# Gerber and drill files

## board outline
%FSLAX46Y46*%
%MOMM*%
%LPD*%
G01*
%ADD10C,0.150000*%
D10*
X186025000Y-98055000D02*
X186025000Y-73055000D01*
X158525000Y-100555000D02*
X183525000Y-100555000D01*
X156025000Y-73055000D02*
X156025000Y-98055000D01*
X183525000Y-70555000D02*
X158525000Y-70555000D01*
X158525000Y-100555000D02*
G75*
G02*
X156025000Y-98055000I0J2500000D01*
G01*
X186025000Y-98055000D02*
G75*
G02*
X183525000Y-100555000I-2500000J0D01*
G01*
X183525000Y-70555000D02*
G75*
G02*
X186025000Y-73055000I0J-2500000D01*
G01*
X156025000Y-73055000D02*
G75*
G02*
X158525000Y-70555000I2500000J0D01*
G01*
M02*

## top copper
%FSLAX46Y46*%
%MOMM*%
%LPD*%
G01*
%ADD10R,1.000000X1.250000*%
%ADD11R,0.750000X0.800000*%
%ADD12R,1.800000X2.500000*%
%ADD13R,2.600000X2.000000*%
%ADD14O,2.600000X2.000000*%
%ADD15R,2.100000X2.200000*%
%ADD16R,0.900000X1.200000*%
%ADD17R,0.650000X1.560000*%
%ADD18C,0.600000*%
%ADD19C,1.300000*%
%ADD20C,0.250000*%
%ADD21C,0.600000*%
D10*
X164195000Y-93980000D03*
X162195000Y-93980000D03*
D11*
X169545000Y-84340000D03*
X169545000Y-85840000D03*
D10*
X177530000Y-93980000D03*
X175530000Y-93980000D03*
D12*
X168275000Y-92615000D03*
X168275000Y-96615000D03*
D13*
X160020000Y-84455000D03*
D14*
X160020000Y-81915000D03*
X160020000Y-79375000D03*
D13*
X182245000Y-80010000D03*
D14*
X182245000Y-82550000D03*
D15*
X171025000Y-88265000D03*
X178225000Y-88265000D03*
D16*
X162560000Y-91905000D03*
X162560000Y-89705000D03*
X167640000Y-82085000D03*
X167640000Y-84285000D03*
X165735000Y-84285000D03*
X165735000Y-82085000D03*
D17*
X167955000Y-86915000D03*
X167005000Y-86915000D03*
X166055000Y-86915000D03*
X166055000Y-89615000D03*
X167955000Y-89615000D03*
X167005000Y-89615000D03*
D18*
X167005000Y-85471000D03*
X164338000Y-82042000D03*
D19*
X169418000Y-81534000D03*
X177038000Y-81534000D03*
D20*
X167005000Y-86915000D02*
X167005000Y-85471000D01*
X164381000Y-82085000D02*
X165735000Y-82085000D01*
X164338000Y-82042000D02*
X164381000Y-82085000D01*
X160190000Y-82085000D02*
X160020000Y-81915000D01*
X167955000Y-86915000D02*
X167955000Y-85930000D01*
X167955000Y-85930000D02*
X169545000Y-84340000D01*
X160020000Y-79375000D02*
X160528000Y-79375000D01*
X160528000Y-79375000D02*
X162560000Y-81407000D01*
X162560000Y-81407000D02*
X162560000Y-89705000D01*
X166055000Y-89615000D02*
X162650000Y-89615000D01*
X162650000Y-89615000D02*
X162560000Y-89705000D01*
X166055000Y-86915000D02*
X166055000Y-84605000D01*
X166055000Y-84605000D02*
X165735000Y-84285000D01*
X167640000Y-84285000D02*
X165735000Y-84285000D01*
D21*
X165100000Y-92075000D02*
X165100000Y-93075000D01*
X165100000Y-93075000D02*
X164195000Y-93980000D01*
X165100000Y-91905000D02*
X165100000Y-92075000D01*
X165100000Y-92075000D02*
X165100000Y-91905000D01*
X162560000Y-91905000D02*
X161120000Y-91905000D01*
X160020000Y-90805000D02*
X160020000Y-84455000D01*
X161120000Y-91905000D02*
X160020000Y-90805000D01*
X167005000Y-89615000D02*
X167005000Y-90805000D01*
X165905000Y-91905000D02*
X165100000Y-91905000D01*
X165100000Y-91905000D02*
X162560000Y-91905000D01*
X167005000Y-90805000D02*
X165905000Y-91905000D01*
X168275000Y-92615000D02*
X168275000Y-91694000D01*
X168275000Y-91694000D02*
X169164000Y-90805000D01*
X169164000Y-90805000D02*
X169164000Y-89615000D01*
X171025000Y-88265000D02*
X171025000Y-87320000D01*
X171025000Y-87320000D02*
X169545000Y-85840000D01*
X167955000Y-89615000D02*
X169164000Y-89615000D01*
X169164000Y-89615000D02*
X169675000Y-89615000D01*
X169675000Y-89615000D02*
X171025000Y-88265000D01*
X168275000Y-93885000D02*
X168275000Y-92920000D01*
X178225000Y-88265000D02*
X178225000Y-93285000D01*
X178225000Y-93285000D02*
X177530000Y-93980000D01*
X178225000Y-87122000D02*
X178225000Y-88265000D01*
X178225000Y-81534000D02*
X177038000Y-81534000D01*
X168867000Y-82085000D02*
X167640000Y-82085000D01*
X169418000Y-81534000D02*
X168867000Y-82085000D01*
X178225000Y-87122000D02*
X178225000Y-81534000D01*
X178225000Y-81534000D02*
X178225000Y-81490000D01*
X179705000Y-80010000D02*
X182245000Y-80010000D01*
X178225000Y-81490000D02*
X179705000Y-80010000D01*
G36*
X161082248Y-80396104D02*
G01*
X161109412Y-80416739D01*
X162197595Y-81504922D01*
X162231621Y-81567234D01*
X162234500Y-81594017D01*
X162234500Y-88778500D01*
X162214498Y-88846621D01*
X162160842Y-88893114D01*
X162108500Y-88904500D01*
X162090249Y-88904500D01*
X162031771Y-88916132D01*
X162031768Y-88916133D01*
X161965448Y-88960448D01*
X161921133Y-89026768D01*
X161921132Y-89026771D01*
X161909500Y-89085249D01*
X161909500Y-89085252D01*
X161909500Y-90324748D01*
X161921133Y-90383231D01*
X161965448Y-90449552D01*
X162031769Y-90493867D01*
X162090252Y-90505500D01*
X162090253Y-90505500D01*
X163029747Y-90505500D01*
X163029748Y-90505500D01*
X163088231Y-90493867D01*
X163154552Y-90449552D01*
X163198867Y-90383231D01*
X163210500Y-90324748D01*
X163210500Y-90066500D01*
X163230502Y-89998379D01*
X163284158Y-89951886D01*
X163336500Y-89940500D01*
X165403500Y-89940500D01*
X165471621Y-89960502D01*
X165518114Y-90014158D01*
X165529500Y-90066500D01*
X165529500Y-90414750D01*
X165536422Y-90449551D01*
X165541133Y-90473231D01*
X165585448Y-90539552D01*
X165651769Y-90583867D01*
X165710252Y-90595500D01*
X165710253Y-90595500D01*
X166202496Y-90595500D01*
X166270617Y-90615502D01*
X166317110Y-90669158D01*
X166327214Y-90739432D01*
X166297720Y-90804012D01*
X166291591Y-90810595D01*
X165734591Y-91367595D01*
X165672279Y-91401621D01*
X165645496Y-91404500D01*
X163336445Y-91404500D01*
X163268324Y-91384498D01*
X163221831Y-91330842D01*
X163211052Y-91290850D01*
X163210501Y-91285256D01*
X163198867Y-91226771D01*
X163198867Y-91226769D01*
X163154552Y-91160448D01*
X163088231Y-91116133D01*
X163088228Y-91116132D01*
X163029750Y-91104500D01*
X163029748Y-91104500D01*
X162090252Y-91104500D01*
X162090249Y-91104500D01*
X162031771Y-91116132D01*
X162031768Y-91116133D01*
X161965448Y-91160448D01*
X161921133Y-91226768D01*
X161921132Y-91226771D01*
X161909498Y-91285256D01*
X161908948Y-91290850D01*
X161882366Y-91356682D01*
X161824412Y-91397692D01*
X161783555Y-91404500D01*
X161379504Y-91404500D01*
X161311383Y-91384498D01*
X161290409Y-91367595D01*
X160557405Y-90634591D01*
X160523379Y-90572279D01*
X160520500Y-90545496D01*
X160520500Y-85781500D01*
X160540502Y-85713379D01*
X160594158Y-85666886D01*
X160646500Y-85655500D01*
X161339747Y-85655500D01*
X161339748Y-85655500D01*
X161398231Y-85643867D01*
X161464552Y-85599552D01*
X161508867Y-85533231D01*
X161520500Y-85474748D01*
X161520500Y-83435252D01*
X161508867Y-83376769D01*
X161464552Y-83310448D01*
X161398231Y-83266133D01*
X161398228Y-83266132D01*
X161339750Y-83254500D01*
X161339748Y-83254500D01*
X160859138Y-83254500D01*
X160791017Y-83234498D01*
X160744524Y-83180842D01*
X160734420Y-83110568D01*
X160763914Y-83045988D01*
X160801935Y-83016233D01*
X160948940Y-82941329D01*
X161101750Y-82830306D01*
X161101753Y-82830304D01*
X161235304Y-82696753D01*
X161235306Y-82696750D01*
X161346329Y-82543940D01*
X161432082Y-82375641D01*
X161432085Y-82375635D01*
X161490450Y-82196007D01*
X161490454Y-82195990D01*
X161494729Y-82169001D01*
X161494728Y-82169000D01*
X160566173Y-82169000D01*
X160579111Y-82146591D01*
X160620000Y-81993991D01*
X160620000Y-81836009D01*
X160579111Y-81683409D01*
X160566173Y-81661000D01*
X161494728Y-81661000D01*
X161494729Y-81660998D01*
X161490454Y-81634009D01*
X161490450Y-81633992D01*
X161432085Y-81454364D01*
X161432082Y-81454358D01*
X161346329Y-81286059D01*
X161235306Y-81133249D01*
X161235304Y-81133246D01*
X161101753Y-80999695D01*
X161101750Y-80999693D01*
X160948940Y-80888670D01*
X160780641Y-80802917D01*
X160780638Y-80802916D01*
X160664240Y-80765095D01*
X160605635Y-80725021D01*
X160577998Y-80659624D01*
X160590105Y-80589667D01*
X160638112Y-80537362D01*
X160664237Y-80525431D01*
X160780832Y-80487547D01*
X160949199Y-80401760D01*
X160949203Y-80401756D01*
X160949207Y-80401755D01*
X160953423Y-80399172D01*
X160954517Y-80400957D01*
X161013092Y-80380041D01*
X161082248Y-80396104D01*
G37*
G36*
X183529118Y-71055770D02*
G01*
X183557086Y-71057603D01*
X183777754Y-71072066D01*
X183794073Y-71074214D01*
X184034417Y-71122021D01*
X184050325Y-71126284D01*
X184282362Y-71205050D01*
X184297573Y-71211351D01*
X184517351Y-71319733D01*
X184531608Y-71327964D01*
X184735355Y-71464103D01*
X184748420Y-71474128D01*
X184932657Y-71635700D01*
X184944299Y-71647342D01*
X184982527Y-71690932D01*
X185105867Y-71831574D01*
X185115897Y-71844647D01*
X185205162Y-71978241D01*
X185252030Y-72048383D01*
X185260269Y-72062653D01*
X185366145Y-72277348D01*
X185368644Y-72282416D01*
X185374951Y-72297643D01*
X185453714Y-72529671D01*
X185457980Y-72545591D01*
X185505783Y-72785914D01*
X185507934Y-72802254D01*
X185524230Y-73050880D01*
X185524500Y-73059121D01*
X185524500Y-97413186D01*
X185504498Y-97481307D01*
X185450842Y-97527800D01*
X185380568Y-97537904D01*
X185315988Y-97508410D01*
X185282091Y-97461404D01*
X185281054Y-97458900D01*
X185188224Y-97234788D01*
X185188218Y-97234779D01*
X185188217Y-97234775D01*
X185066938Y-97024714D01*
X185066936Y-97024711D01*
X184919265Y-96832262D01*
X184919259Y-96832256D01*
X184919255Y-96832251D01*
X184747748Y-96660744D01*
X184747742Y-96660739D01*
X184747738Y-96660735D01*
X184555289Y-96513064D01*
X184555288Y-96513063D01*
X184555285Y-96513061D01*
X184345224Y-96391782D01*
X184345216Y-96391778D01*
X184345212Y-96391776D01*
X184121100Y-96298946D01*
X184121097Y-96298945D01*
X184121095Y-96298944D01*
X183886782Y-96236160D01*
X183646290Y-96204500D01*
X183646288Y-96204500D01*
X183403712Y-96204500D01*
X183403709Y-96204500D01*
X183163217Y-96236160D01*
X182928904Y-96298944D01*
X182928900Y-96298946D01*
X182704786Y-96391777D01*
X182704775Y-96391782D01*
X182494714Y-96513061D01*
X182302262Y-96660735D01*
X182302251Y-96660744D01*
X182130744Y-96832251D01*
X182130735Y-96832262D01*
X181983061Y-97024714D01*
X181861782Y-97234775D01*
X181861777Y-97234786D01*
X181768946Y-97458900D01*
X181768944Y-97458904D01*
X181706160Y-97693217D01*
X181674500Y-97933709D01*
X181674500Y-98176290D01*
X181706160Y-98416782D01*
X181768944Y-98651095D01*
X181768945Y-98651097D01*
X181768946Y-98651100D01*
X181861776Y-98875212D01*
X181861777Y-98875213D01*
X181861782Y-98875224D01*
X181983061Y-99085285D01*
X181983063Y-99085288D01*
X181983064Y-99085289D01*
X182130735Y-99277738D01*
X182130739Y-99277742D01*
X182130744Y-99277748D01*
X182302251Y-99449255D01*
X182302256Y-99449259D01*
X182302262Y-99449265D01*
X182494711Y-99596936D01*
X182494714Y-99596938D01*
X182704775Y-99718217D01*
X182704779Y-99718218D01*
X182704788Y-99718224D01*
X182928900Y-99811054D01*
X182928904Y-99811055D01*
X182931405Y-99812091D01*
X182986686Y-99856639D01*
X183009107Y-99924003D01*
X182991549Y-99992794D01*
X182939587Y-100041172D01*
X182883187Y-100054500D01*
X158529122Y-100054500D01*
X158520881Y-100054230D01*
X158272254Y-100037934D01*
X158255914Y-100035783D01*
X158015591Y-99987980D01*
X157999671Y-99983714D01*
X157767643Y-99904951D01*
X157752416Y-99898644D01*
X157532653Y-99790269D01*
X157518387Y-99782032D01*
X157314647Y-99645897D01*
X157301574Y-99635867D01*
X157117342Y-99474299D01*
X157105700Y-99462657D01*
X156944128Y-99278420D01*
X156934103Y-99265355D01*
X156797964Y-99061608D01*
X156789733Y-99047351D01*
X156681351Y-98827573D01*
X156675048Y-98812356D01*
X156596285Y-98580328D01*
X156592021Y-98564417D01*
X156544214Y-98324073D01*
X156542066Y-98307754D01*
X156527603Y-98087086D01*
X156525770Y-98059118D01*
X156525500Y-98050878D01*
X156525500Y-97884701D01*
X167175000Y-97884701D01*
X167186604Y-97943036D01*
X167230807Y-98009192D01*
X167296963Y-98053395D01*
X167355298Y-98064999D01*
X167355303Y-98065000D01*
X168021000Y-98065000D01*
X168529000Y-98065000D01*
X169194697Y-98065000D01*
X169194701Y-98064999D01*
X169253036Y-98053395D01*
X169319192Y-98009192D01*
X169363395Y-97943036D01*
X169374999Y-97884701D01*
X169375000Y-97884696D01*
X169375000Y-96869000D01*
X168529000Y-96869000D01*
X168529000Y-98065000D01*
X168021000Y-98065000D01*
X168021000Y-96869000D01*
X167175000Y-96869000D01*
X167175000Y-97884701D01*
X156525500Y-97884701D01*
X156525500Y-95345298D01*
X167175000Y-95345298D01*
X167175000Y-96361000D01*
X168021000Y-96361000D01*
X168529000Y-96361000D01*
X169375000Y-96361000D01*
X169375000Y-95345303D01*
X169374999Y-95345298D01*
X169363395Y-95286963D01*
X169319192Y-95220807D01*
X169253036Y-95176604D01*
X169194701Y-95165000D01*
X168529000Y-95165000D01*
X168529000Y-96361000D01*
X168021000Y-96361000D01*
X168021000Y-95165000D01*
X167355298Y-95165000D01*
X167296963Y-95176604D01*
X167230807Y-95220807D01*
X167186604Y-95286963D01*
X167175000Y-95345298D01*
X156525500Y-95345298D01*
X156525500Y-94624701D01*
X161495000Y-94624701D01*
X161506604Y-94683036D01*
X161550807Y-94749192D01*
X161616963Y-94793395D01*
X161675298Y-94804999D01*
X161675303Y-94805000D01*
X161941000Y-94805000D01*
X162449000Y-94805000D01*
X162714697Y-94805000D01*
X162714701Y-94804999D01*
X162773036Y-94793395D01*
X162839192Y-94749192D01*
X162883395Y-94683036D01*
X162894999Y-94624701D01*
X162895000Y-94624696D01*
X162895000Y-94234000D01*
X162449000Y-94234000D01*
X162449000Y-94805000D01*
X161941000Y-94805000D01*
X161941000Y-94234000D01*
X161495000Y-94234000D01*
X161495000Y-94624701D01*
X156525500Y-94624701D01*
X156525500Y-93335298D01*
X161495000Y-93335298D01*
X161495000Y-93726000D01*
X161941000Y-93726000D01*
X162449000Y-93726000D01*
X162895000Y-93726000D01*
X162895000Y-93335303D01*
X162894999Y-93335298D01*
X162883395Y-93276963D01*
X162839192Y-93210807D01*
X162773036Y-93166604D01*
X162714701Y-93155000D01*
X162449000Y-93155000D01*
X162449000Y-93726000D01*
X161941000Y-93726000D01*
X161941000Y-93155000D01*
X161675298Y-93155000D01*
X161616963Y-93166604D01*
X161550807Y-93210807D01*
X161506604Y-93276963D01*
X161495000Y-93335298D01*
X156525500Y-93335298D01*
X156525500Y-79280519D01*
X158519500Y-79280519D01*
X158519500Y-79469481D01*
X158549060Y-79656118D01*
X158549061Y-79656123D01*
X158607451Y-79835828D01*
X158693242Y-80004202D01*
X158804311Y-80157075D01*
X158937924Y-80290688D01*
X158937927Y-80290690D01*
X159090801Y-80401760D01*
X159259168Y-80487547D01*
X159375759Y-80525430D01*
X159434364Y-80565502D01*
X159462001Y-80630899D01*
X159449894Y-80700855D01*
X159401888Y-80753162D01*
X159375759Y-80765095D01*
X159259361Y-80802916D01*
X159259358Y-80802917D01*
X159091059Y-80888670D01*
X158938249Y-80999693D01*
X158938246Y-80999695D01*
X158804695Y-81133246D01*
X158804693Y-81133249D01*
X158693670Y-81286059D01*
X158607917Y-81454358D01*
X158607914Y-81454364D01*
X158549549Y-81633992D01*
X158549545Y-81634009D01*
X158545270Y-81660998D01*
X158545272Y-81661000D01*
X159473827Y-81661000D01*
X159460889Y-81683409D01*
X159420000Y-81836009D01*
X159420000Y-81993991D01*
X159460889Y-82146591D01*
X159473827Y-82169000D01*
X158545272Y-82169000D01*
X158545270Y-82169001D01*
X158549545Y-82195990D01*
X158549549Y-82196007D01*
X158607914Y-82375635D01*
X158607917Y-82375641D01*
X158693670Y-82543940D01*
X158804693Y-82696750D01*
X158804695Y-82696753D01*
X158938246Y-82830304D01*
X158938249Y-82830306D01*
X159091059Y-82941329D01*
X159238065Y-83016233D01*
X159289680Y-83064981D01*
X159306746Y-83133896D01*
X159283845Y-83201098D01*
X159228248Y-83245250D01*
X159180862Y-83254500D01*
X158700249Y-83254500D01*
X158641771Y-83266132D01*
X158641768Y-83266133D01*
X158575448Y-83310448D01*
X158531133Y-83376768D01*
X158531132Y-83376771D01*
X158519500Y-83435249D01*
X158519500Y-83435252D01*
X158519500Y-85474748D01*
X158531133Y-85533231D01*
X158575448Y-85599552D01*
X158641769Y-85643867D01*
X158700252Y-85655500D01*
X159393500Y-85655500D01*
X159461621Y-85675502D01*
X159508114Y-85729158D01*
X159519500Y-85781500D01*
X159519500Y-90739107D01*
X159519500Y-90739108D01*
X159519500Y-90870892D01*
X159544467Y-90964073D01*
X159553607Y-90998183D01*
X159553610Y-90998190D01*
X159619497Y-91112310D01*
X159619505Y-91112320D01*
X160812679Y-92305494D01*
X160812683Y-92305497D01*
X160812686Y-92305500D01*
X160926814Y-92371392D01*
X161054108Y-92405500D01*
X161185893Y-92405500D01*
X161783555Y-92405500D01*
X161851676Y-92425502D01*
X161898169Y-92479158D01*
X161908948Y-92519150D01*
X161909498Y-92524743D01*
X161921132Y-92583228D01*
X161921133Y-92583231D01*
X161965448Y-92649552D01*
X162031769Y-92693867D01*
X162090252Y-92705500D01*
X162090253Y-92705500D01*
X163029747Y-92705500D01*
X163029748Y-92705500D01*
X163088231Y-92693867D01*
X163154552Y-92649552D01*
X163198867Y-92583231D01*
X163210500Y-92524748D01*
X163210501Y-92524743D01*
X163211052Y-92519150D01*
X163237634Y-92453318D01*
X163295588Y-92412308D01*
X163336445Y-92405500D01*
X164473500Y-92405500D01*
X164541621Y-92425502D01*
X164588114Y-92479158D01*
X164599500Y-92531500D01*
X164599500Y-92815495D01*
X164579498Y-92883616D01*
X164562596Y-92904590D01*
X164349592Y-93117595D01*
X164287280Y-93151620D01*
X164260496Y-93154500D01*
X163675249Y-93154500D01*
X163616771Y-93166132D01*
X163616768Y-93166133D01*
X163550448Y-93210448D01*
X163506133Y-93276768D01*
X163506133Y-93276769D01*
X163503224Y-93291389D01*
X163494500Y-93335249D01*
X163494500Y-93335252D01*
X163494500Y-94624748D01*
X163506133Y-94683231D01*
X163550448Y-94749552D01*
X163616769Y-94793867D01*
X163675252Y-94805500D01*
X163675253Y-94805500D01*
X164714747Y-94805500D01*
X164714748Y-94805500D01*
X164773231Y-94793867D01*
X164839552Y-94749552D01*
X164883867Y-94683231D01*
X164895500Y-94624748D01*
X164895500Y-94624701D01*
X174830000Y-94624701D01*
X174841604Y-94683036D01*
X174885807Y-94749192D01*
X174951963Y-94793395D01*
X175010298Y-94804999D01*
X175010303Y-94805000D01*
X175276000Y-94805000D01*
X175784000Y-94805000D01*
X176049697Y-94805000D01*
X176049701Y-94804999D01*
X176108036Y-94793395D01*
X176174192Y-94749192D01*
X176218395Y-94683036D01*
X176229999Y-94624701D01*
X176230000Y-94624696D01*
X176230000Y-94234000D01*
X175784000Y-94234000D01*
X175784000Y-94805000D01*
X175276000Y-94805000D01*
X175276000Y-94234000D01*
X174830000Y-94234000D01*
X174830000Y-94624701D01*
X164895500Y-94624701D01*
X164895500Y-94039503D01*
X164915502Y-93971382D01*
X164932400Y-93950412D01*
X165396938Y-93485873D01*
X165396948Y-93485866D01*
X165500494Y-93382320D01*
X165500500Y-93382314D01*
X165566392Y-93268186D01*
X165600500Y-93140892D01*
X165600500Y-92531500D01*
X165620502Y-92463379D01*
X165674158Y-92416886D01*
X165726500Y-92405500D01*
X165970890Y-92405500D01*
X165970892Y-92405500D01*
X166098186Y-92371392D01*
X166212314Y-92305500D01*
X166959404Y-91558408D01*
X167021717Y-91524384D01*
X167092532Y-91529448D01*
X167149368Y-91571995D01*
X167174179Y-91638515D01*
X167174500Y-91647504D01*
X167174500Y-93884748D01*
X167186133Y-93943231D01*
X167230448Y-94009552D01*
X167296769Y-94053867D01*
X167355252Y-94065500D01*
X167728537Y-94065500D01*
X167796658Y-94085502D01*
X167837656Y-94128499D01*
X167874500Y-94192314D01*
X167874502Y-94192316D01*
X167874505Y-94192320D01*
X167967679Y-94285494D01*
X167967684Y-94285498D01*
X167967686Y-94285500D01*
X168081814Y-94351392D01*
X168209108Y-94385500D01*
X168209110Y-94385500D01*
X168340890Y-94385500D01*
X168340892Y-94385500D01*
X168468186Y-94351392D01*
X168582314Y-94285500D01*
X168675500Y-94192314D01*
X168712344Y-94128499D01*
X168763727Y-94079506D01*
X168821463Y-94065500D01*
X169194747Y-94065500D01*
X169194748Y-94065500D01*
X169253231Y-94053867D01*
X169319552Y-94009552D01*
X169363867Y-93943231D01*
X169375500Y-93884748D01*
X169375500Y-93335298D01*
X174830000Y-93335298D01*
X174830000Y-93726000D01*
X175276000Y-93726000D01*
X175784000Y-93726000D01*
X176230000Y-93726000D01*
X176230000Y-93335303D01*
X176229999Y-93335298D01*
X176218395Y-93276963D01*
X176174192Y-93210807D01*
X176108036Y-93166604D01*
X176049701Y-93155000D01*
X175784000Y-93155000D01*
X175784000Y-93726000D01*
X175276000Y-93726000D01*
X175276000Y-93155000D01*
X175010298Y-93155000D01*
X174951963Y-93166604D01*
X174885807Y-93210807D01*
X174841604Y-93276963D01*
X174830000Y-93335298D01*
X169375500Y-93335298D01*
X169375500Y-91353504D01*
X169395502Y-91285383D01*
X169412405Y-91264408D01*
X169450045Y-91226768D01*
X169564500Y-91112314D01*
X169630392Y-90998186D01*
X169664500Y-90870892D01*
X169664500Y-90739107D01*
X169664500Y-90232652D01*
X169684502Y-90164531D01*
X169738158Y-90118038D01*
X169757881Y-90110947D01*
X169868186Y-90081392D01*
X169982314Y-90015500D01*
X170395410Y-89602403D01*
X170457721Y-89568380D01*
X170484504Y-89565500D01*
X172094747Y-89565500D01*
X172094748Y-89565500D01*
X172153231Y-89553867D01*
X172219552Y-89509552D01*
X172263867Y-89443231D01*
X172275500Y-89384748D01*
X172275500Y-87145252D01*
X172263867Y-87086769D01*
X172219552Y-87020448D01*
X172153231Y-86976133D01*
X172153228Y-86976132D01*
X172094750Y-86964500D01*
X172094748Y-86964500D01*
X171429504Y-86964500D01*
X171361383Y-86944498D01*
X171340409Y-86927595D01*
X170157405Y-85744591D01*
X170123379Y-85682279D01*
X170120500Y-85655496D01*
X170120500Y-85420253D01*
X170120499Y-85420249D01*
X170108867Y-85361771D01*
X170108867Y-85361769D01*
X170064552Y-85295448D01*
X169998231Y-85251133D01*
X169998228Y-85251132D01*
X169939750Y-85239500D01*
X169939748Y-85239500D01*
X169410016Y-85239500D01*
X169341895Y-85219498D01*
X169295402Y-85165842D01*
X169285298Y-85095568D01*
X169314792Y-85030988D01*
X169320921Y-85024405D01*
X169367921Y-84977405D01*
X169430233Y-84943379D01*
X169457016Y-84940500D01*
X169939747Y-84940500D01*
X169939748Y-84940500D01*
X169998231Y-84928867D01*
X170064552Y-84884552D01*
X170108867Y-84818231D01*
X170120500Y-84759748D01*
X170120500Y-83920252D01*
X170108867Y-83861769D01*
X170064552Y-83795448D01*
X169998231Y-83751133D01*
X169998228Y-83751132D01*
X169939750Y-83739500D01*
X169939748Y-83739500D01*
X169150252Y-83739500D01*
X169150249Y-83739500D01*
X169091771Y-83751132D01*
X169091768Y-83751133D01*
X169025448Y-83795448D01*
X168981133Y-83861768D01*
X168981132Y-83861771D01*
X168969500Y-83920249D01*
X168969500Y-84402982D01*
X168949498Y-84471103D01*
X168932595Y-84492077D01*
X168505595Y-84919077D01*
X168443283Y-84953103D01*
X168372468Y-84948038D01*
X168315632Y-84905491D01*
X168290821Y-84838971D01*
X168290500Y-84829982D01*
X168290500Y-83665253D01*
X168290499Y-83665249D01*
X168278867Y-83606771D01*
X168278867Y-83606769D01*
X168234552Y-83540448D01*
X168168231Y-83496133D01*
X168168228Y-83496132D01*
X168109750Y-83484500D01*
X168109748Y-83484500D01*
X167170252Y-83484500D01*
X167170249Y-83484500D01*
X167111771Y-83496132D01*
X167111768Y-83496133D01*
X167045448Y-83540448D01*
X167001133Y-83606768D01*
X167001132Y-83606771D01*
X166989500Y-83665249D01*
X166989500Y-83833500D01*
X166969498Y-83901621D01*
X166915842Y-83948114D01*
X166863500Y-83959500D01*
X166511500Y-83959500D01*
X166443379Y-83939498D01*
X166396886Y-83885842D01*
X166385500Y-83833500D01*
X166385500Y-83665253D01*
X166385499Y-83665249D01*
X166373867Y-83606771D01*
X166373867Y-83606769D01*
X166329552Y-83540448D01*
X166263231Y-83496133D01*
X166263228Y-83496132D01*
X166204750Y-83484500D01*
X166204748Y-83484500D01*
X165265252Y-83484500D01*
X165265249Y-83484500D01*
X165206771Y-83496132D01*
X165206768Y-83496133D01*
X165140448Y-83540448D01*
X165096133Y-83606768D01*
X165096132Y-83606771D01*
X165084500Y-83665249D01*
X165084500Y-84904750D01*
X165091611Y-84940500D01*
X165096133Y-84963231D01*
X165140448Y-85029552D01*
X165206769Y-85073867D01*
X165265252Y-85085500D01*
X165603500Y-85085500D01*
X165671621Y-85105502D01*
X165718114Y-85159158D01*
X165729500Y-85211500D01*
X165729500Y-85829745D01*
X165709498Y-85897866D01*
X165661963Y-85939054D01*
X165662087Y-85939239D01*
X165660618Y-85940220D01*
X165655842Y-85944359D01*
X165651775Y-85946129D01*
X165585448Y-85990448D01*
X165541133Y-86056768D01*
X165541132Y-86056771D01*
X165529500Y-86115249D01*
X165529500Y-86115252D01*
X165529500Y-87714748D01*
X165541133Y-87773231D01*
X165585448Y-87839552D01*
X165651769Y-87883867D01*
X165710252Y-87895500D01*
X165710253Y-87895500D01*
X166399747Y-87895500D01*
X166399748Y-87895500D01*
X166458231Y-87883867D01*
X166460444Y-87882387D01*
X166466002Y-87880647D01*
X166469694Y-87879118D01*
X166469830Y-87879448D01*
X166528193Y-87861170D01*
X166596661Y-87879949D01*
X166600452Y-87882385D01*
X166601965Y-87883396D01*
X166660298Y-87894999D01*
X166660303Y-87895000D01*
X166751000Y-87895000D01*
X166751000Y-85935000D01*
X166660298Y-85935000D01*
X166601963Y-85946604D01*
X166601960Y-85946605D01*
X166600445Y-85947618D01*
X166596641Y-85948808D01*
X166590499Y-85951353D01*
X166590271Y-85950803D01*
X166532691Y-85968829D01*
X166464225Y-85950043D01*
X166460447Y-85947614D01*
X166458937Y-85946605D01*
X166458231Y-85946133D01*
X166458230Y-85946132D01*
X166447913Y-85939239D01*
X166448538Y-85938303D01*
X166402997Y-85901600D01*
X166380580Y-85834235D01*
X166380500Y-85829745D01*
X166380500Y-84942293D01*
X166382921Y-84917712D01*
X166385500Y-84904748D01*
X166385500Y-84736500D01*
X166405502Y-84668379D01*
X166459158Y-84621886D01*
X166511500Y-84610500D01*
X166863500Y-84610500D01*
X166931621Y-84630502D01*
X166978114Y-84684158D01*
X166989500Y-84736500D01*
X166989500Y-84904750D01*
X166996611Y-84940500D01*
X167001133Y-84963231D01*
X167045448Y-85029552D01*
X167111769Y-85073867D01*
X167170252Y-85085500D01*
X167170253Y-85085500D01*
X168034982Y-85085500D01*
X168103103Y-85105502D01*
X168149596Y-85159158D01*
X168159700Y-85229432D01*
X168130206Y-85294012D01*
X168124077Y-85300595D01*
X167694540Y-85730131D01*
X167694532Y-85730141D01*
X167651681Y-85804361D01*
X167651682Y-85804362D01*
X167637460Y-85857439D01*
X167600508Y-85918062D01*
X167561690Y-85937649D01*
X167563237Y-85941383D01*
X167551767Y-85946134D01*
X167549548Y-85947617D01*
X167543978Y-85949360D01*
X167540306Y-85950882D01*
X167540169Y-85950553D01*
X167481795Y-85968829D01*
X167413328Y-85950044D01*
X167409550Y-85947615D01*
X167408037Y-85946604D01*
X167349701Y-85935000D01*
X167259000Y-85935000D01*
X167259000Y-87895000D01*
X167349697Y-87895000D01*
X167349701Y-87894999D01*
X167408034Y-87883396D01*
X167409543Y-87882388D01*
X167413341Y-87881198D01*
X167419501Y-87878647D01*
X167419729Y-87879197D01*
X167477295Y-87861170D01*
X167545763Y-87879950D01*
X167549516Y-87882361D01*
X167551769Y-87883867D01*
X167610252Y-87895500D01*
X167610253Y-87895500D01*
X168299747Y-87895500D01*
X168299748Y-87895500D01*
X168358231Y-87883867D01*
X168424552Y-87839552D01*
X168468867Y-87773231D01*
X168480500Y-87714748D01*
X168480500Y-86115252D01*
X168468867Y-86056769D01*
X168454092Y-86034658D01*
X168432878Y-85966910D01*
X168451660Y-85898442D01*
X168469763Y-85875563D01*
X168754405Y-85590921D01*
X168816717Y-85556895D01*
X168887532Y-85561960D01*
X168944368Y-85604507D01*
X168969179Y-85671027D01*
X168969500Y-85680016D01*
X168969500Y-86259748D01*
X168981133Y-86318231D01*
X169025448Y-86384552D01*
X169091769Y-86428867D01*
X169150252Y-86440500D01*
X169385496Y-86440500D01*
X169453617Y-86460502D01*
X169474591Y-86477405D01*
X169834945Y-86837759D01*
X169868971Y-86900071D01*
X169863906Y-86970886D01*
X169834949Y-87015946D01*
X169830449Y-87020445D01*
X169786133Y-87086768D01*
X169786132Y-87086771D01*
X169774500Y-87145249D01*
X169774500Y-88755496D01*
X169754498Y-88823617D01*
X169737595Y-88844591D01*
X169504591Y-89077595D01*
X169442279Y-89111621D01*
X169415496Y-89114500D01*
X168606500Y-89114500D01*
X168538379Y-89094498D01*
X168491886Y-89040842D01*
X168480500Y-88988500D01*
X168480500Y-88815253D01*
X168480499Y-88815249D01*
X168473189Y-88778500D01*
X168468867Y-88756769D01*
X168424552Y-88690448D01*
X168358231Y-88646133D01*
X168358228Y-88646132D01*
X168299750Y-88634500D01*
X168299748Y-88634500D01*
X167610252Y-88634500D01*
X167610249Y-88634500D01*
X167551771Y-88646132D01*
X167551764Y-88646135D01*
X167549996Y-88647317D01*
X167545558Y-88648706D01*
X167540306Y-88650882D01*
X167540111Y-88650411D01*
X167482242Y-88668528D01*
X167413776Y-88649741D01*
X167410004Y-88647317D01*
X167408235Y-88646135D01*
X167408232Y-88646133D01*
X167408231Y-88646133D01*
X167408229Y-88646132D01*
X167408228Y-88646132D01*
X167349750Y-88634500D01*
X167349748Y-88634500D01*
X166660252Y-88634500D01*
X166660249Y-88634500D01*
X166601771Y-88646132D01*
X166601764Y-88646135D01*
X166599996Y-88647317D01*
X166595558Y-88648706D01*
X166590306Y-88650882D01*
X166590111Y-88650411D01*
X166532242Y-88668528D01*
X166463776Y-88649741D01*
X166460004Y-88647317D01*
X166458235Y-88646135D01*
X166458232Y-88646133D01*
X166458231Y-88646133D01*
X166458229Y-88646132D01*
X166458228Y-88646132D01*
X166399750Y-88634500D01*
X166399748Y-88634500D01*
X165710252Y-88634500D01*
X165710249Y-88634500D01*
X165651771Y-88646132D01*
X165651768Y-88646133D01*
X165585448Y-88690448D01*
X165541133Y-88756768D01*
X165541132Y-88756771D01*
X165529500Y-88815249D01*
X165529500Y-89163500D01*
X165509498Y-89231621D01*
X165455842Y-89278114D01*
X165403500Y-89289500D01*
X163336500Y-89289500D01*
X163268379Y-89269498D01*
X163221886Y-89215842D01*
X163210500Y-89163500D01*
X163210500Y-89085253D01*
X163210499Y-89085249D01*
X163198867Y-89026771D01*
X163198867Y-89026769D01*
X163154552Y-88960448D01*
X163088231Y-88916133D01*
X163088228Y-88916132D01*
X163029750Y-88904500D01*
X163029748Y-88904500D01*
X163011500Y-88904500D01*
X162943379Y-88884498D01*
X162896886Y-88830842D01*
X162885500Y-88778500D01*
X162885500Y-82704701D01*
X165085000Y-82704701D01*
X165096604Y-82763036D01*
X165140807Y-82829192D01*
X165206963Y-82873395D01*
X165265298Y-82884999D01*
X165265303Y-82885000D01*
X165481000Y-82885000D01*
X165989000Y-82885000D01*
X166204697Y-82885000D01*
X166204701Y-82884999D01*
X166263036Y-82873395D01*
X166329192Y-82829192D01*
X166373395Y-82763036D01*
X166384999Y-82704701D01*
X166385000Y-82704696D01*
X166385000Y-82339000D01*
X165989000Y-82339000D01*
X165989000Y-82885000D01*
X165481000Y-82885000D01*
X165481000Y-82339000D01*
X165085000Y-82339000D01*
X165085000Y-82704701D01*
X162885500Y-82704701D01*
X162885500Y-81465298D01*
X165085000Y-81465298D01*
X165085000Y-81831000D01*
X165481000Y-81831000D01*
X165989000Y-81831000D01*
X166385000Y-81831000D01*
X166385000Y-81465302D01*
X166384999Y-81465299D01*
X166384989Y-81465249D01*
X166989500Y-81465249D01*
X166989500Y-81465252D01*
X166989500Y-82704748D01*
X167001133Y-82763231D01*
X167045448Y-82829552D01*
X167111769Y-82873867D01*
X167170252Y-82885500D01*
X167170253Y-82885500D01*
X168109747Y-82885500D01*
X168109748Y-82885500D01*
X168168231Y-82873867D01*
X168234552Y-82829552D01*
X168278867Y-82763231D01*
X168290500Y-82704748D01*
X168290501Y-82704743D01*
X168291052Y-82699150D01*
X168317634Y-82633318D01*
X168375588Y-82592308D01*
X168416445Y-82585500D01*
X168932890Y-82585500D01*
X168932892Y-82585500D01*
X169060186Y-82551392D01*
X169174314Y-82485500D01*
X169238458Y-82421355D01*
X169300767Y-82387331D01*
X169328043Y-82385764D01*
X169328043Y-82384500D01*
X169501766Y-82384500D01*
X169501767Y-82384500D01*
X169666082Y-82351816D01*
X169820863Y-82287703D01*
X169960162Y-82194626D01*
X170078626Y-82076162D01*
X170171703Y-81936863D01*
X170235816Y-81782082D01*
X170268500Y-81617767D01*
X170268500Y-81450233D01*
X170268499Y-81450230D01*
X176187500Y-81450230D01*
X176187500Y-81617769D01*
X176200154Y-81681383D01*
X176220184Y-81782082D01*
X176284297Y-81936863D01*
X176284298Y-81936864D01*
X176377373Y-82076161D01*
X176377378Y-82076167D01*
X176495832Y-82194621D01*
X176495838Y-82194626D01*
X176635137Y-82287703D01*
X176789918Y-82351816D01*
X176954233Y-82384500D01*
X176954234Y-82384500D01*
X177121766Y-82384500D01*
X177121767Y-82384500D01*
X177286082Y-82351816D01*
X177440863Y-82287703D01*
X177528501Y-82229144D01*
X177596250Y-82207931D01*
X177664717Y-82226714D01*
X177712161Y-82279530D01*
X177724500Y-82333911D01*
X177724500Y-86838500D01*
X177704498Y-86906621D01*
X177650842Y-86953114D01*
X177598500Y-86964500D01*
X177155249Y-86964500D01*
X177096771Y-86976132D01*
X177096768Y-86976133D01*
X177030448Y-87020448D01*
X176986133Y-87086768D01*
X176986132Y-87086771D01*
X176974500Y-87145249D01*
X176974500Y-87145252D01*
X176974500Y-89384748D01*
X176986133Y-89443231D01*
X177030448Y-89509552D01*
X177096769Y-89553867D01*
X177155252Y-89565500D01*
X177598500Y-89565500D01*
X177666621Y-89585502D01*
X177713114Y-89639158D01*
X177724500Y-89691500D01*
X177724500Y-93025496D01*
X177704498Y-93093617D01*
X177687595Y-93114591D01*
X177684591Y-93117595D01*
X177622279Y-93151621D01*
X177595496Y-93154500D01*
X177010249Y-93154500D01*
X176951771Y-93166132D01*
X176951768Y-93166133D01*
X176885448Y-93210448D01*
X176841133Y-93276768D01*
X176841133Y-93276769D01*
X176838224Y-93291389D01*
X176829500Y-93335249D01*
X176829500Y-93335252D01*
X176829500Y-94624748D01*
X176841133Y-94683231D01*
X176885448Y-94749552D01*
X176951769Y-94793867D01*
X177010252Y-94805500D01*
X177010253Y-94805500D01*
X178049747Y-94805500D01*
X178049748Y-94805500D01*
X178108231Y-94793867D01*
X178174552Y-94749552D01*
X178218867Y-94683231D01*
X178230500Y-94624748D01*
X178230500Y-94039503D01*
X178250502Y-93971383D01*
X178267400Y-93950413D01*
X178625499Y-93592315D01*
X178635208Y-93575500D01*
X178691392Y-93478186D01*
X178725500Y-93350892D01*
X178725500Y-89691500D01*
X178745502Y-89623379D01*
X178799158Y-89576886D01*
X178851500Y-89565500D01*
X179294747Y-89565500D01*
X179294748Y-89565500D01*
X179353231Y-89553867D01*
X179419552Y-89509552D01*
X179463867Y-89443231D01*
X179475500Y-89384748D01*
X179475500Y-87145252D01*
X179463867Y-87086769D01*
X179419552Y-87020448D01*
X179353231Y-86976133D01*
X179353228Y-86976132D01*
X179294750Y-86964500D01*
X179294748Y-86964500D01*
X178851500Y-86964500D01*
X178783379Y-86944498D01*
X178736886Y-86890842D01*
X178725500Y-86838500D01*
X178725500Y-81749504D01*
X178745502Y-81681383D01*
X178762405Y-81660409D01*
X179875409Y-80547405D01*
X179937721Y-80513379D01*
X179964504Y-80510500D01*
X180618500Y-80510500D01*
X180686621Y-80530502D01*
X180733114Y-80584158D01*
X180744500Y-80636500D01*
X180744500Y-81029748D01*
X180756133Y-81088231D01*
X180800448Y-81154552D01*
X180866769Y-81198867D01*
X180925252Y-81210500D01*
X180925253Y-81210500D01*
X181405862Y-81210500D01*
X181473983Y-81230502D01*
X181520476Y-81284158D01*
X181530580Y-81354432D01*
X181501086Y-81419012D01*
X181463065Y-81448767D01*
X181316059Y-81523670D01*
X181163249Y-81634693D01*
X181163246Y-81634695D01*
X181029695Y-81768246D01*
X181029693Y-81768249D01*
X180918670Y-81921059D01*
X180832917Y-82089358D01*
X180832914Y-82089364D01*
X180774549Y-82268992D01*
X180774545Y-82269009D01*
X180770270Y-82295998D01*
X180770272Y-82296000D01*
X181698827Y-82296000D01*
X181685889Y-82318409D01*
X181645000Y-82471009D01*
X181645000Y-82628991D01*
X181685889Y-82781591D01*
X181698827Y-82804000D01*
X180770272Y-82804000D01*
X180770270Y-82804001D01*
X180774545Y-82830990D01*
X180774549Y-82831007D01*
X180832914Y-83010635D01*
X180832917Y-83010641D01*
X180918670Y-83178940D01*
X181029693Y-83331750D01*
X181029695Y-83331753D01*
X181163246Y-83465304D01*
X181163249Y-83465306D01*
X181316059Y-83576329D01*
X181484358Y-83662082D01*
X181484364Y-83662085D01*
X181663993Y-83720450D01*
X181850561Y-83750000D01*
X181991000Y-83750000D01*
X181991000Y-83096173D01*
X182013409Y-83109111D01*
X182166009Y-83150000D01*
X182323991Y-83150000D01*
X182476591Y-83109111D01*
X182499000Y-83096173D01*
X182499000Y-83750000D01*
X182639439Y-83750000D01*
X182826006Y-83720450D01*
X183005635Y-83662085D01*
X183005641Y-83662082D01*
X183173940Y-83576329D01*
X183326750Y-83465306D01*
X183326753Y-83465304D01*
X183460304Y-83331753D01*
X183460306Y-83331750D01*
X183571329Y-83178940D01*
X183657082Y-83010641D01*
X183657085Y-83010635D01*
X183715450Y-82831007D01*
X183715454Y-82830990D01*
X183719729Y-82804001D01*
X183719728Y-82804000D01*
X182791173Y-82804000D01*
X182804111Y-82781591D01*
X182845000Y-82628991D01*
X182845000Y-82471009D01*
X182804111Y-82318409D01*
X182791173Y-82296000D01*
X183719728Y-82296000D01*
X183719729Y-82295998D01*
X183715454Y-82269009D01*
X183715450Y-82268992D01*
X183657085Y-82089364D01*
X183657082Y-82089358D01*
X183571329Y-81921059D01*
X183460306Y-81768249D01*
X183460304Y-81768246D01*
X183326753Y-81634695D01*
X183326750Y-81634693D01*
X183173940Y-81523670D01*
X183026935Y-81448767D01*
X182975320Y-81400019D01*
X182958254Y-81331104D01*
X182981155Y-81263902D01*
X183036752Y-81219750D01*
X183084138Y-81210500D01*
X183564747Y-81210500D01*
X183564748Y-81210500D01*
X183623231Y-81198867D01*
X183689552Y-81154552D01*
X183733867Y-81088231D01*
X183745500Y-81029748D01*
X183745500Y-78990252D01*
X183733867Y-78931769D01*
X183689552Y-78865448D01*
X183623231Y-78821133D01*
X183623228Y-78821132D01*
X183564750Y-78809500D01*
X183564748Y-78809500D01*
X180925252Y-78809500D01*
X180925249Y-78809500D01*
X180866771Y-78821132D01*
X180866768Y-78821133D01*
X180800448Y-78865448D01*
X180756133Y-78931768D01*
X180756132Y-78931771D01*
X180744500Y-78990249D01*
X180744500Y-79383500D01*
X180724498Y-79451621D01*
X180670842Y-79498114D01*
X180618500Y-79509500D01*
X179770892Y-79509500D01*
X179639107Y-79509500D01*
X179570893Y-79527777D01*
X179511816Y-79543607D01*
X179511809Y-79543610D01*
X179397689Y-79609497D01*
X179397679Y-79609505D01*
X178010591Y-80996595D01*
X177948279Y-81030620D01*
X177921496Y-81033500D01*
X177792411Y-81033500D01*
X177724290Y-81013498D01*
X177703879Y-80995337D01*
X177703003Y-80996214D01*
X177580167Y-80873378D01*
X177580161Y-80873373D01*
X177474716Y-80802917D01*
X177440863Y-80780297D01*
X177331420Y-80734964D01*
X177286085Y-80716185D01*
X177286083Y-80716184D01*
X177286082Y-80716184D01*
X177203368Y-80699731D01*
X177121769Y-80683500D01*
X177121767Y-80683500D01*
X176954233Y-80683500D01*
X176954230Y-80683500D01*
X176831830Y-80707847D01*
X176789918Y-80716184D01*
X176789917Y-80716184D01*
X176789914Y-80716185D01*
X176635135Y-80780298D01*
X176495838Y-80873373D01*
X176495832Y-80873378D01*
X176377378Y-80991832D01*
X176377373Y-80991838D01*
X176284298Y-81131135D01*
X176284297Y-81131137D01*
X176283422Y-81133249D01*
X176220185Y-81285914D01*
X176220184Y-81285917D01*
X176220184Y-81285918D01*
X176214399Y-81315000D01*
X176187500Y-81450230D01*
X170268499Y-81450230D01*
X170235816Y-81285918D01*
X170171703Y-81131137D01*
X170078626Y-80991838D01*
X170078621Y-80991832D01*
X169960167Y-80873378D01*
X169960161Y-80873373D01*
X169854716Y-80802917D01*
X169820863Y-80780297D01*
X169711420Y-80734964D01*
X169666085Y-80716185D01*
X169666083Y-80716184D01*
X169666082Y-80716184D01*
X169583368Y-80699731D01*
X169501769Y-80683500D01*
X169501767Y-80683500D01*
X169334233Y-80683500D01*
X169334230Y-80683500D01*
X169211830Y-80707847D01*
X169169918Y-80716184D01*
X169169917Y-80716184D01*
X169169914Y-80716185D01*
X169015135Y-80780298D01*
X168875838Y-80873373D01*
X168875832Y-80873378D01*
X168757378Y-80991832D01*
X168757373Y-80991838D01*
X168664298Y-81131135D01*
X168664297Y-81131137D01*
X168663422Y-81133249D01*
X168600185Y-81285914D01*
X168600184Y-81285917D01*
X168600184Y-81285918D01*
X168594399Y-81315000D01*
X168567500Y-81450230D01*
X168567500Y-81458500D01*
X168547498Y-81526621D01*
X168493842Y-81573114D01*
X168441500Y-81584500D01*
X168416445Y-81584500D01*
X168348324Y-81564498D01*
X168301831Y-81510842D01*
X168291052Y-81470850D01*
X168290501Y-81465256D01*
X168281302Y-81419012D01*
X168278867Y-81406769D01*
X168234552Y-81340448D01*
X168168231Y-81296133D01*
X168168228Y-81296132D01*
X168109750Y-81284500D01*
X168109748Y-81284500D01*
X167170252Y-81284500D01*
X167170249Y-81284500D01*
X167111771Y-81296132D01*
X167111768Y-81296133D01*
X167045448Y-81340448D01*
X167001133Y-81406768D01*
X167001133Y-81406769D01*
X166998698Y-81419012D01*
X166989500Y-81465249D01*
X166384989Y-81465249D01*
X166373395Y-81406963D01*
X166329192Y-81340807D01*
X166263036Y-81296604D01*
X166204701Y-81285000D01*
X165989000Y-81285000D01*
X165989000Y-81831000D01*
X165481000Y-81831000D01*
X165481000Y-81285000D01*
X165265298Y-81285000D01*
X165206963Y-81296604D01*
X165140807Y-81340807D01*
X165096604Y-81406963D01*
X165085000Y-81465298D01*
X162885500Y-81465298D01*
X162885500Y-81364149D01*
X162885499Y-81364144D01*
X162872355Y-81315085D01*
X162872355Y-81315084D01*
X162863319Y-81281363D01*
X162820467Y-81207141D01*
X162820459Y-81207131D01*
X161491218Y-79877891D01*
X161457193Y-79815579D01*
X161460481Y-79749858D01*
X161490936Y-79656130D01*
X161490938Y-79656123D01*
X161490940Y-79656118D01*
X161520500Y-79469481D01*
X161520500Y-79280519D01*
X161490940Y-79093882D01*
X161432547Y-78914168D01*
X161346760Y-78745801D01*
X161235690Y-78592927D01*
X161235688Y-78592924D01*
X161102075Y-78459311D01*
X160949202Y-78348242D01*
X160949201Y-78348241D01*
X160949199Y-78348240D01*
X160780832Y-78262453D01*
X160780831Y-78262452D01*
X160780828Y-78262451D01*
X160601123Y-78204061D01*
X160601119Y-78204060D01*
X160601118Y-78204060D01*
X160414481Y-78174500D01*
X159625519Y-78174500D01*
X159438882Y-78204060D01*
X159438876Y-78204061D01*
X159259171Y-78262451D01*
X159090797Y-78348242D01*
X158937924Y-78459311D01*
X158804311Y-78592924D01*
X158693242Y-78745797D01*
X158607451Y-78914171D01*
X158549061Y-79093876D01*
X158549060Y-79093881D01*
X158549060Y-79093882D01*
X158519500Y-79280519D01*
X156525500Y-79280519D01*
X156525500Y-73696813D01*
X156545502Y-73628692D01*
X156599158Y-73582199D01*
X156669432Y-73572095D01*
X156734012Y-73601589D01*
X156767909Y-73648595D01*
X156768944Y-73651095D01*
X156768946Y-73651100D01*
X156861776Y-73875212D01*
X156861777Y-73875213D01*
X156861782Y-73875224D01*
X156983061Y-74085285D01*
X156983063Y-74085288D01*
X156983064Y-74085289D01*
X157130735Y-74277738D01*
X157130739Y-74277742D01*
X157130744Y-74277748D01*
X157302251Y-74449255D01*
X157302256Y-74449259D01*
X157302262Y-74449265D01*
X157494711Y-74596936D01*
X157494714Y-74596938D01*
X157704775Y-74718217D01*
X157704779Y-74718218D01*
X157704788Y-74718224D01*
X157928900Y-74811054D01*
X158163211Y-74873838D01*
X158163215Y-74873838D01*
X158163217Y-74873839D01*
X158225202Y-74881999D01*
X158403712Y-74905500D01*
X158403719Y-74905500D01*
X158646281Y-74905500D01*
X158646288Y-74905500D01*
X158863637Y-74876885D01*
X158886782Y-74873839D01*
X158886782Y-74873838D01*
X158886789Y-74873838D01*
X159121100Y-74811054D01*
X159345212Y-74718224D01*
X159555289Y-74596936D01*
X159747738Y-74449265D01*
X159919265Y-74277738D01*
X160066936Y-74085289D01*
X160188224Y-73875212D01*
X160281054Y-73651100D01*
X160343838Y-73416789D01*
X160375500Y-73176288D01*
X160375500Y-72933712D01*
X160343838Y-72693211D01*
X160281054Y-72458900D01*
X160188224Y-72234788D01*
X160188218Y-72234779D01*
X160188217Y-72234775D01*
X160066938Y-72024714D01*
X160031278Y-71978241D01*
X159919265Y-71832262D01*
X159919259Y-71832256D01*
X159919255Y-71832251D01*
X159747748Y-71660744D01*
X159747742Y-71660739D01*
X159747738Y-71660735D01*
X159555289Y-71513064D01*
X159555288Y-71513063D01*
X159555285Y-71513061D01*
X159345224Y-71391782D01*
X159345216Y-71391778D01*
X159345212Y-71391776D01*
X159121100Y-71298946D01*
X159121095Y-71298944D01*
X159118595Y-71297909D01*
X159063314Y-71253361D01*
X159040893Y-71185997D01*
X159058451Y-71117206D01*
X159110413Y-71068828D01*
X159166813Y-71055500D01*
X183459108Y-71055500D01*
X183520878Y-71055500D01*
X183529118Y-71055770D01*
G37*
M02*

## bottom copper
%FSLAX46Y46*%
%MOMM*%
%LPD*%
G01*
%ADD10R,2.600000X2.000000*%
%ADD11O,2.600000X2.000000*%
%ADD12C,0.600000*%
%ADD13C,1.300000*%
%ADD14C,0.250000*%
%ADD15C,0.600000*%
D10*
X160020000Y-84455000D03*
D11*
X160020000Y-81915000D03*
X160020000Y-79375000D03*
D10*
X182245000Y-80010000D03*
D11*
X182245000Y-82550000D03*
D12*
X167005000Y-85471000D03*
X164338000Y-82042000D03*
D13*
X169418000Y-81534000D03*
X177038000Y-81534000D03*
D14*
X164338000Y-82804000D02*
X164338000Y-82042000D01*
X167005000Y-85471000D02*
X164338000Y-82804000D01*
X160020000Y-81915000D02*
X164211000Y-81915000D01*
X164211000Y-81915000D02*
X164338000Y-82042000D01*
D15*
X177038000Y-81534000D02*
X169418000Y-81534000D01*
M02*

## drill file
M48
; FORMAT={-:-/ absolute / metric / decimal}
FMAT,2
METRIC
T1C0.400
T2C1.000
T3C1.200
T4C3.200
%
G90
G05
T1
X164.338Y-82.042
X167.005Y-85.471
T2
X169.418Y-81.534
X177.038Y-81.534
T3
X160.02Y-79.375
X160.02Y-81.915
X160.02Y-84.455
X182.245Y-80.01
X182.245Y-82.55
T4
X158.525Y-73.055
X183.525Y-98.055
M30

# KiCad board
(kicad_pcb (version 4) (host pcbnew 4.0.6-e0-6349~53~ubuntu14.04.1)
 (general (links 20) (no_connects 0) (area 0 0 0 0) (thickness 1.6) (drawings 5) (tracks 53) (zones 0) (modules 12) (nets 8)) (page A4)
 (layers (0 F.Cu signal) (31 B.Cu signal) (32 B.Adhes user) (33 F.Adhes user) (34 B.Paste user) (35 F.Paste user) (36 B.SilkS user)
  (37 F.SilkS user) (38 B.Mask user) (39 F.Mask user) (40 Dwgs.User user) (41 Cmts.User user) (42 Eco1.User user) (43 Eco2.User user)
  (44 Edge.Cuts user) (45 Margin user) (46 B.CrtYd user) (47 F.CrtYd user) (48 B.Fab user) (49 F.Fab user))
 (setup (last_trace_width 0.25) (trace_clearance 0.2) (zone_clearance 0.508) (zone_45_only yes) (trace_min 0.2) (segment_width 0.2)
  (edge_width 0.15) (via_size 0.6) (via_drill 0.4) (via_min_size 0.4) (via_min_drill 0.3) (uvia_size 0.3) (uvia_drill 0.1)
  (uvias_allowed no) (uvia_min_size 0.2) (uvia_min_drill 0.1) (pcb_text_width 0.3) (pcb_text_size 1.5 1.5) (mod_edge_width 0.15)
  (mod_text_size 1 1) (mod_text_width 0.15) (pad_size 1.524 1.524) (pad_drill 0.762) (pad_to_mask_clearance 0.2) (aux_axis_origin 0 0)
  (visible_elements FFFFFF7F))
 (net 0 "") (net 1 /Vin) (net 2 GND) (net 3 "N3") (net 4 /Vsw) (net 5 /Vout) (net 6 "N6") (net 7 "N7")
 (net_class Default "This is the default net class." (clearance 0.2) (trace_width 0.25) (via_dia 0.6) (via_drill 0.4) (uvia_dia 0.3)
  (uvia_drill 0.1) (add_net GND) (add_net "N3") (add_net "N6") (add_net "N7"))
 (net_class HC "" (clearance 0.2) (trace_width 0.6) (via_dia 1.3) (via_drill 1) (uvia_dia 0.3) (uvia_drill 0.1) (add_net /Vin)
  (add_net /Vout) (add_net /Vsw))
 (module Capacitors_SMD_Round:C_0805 (layer F.Cu) (at 163.195 93.98 180)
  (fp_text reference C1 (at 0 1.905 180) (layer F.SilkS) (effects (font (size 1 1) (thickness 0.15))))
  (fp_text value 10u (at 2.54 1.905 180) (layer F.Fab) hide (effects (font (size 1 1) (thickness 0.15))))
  (pad 1 smd rect (at -1 0 180) (size 1 1.25) (layers F.Cu F.Paste F.Mask) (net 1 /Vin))
  (pad 2 smd rect (at 1 0 180) (size 1 1.25) (layers F.Cu F.Paste F.Mask) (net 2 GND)))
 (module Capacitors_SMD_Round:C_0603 (layer F.Cu) (at 169.545 85.09 270)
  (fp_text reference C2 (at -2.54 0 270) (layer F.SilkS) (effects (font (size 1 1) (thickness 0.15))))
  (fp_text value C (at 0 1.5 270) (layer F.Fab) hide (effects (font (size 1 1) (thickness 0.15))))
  (pad 1 smd rect (at -0.75 0 270) (size 0.8 0.75) (layers F.Cu F.Paste F.Mask) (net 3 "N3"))
  (pad 2 smd rect (at 0.75 0 270) (size 0.8 0.75) (layers F.Cu F.Paste F.Mask) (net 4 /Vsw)))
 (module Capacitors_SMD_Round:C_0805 (layer F.Cu) (at 176.53 93.98 180)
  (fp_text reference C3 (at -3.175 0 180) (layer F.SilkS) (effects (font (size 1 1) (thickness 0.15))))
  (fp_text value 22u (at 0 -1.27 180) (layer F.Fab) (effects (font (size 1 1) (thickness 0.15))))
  (pad 1 smd rect (at -1 0 180) (size 1 1.25) (layers F.Cu F.Paste F.Mask) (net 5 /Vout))
  (pad 2 smd rect (at 1 0 180) (size 1 1.25) (layers F.Cu F.Paste F.Mask) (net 2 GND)))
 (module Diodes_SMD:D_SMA (layer F.Cu) (at 168.275 94.615 270)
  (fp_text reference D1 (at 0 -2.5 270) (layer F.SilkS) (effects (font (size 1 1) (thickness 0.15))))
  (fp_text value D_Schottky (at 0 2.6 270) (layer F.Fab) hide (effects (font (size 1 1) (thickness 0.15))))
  (pad 1 smd rect (at -2 0 270) (size 2.5 1.8) (layers F.Cu F.Paste F.Mask) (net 4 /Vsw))
  (pad 2 smd rect (at 2 0 270) (size 2.5 1.8) (layers F.Cu F.Paste F.Mask) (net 2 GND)))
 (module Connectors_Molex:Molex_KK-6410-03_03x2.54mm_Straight (layer F.Cu) (at 160.02 84.455 90)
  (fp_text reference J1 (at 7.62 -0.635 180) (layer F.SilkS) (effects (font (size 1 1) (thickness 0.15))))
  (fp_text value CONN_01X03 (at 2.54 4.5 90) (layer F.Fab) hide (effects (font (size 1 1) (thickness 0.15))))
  (pad 1 thru_hole rect (at 0 0 90) (size 2 2.6) (drill 1.2) (layers *.Cu *.Mask) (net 1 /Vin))
  (pad 2 thru_hole oval (at 2.54 0 90) (size 2 2.6) (drill 1.2) (layers *.Cu *.Mask) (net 2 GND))
  (pad 3 thru_hole oval (at 5.08 0 90) (size 2 2.6) (drill 1.2) (layers *.Cu *.Mask) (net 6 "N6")))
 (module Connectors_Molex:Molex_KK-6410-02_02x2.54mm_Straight (layer F.Cu) (at 182.245 80.01 270)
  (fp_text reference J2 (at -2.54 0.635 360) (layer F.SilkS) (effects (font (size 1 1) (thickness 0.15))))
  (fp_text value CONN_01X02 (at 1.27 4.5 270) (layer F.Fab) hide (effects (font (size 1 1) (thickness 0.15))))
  (pad 1 thru_hole rect (at 0 0 270) (size 2 2.6) (drill 1.2) (layers *.Cu *.Mask) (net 5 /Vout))
  (pad 2 thru_hole oval (at 2.54 0 270) (size 2 2.6) (drill 1.2) (layers *.Cu *.Mask) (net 2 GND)))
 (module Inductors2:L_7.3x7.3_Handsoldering (layer F.Cu) (at 174.625 88.265)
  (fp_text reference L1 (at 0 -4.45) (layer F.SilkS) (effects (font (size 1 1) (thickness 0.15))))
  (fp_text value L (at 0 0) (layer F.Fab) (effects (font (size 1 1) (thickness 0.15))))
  (pad 1 smd rect (at -3.6 0) (size 2.1 2.2) (layers F.Cu F.Paste F.Mask) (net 4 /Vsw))
  (pad 2 smd rect (at 3.6 0) (size 2.1 2.2) (layers F.Cu F.Paste F.Mask) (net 5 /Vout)))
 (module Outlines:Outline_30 (layer F.Cu) (at 156.025 70.555)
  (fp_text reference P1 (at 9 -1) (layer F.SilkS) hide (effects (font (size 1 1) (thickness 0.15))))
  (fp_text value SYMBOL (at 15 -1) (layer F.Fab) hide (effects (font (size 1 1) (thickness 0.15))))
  (fp_line (start 30 27.5) (end 30 2.5) (layer Edge.Cuts) (width 0.15))
  (fp_line (start 2.5 30) (end 27.5 30) (layer Edge.Cuts) (width 0.15))
  (fp_line (start 0 2.5) (end 0 27.5) (layer Edge.Cuts) (width 0.15))
  (fp_line (start 27.5 0) (end 2.5 0) (layer Edge.Cuts) (width 0.15))
  (fp_arc (start 2.5 27.5) (end 2.5 30) (angle 90) (layer Edge.Cuts) (width 0.15))
  (fp_arc (start 27.5 27.5) (end 30 27.5) (angle 90) (layer Edge.Cuts) (width 0.15))
  (fp_arc (start 27.5 2.5) (end 27.5 0) (angle 90) (layer Edge.Cuts) (width 0.15))
  (fp_arc (start 2.5 2.5) (end 0 2.5) (angle 90) (layer Edge.Cuts) (width 0.15))
  (pad "" np_thru_hole circle (at 2.5 2.5) (size 3.2 3.2) (drill 3.2) (layers *.Cu *.Mask))
  (pad "" np_thru_hole circle (at 27.5 27.5) (size 3.2 3.2) (drill 3.2) (layers *.Cu *.Mask)))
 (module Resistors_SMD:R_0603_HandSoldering (layer F.Cu) (at 162.56 90.805 90)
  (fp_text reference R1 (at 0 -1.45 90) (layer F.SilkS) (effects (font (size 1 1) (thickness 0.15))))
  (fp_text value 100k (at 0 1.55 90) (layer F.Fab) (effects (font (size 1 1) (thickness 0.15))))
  (pad 1 smd rect (at -1.1 0 90) (size 1.2 0.9) (layers F.Cu F.Paste F.Mask) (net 1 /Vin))
  (pad 2 smd rect (at 1.1 0 90) (size 1.2 0.9) (layers F.Cu F.Paste F.Mask) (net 6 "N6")))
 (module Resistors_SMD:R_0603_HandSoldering (layer F.Cu) (at 167.64 83.185 270)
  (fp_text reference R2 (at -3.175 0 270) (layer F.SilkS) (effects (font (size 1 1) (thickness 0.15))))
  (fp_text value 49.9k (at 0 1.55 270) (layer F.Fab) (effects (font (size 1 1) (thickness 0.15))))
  (pad 1 smd rect (at -1.1 0 270) (size 1.2 0.9) (layers F.Cu F.Paste F.Mask) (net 5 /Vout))
  (pad 2 smd rect (at 1.1 0 270) (size 1.2 0.9) (layers F.Cu F.Paste F.Mask) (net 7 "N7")))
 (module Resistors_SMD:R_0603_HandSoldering (layer F.Cu) (at 165.735 83.185 90)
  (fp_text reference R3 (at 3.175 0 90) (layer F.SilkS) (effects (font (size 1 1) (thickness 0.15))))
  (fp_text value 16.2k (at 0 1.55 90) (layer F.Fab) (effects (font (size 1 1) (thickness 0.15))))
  (pad 1 smd rect (at -1.1 0 90) (size 1.2 0.9) (layers F.Cu F.Paste F.Mask) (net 7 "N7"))
  (pad 2 smd rect (at 1.1 0 90) (size 1.2 0.9) (layers F.Cu F.Paste F.Mask) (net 2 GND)))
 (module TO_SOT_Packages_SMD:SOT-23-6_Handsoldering (layer F.Cu) (at 167.005 88.265 270)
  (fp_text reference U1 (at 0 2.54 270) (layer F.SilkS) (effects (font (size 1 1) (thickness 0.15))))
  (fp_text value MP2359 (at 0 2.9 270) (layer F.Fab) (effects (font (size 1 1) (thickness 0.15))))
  (pad 1 smd rect (at -1.35 -0.95 270) (size 1.56 0.65) (layers F.Cu F.Paste F.Mask) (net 3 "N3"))
  (pad 2 smd rect (at -1.35 0 270) (size 1.56 0.65) (layers F.Cu F.Paste F.Mask) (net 2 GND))
  (pad 3 smd rect (at -1.35 0.95 270) (size 1.56 0.65) (layers F.Cu F.Paste F.Mask) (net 7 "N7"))
  (pad 4 smd rect (at 1.35 0.95 270) (size 1.56 0.65) (layers F.Cu F.Paste F.Mask) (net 6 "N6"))
  (pad 6 smd rect (at 1.35 -0.95 270) (size 1.56 0.65) (layers F.Cu F.Paste F.Mask) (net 4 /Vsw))
  (pad 5 smd rect (at 1.35 0 270) (size 1.56 0.65) (layers F.Cu F.Paste F.Mask) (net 1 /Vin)))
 (segment (start 167.005 86.915) (end 167.005 85.471) (width 0.25) (layer F.Cu) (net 2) (status 400000))
 (segment (start 164.338 82.804) (end 164.338 82.042) (width 0.25) (layer B.Cu) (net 2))
 (segment (start 167.005 85.471) (end 164.338 82.804) (width 0.25) (layer B.Cu) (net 2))
 (via (at 167.005 85.471) (size 0.6) (drill 0.4) (layers F.Cu B.Cu) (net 2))
 (segment (start 160.02 81.915) (end 164.211 81.915) (width 0.25) (layer B.Cu) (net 2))
 (segment (start 164.381 82.085) (end 165.735 82.085) (width 0.25) (layer F.Cu) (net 2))
 (segment (start 164.338 82.042) (end 164.381 82.085) (width 0.25) (layer F.Cu) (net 2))
 (via (at 164.338 82.042) (size 0.6) (drill 0.4) (layers F.Cu B.Cu) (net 2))
 (segment (start 164.211 81.915) (end 164.338 82.042) (width 0.25) (layer B.Cu) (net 2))
 (segment (start 160.19 82.085) (end 160.02 81.915) (width 0.25) (layer F.Cu) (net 2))
 (segment (start 167.955 86.915) (end 167.955 85.93) (width 0.25) (layer F.Cu) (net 3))
 (segment (start 167.955 85.93) (end 169.545 84.34) (width 0.25) (layer F.Cu) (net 3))
 (segment (start 160.02 79.375) (end 160.528 79.375) (width 0.25) (layer F.Cu) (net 6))
 (segment (start 160.528 79.375) (end 162.56 81.407) (width 0.25) (layer F.Cu) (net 6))
 (segment (start 162.56 81.407) (end 162.56 89.705) (width 0.25) (layer F.Cu) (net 6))
 (segment (start 166.055 89.615) (end 162.65 89.615) (width 0.25) (layer F.Cu) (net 6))
 (segment (start 162.65 89.615) (end 162.56 89.705) (width 0.25) (layer F.Cu) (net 6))
 (segment (start 166.055 86.915) (end 166.055 84.605) (width 0.25) (layer F.Cu) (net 7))
 (segment (start 166.055 84.605) (end 165.735 84.285) (width 0.25) (layer F.Cu) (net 7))
 (segment (start 167.64 84.285) (end 165.735 84.285) (width 0.25) (layer F.Cu) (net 7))
 (segment (start 165.1 92.075) (end 165.1 93.075) (width 0.6) (layer F.Cu) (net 1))
 (segment (start 165.1 93.075) (end 164.195 93.98) (width 0.6) (layer F.Cu) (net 1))
 (segment (start 165.1 91.905) (end 165.1 92.075) (width 0.6) (layer F.Cu) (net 1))
 (segment (start 165.1 92.075) (end 165.1 91.905) (width 0.6) (layer F.Cu) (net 1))
 (segment (start 162.56 91.905) (end 161.12 91.905) (width 0.6) (layer F.Cu) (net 1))
 (segment (start 160.02 90.805) (end 160.02 84.455) (width 0.6) (layer F.Cu) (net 1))
 (segment (start 161.12 91.905) (end 160.02 90.805) (width 0.6) (layer F.Cu) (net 1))
 (segment (start 167.005 89.615) (end 167.005 90.805) (width 0.6) (layer F.Cu) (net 1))
 (segment (start 165.905 91.905) (end 165.1 91.905) (width 0.6) (layer F.Cu) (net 1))
 (segment (start 165.1 91.905) (end 162.56 91.905) (width 0.6) (layer F.Cu) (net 1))
 (segment (start 167.005 90.805) (end 165.905 91.905) (width 0.6) (layer F.Cu) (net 1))
 (segment (start 168.275 92.615) (end 168.275 91.694) (width 0.6) (layer F.Cu) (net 4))
 (segment (start 168.275 91.694) (end 169.164 90.805) (width 0.6) (layer F.Cu) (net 4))
 (segment (start 169.164 90.805) (end 169.164 89.615) (width 0.6) (layer F.Cu) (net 4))
 (segment (start 171.025 88.265) (end 171.025 87.32) (width 0.6) (layer F.Cu) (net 4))
 (segment (start 171.025 87.32) (end 169.545 85.84) (width 0.6) (layer F.Cu) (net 4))
 (segment (start 167.955 89.615) (end 169.164 89.615) (width 0.6) (layer F.Cu) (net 4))
 (segment (start 169.164 89.615) (end 169.675 89.615) (width 0.6) (layer F.Cu) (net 4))
 (segment (start 169.675 89.615) (end 171.025 88.265) (width 0.6) (layer F.Cu) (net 4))
 (segment (start 168.275 93.885) (end 168.275 92.92) (width 0.6) (layer F.Cu) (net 4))
 (segment (start 178.225 88.265) (end 178.225 93.285) (width 0.6) (layer F.Cu) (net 5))
 (segment (start 178.225 93.285) (end 177.53 93.98) (width 0.6) (layer F.Cu) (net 5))
 (segment (start 178.225 87.122) (end 178.225 88.265) (width 0.6) (layer F.Cu) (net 5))
 (segment (start 178.225 81.534) (end 177.038 81.534) (width 0.6) (layer F.Cu) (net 5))
 (segment (start 168.867 82.085) (end 167.64 82.085) (width 0.6) (layer F.Cu) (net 5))
 (segment (start 169.418 81.534) (end 168.867 82.085) (width 0.6) (layer F.Cu) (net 5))
 (via (at 169.418 81.534) (size 1.3) (drill 1) (layers F.Cu B.Cu) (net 5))
 (segment (start 177.038 81.534) (end 169.418 81.534) (width 0.6) (layer B.Cu) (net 5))
 (via (at 177.038 81.534) (size 1.3) (drill 1) (layers F.Cu B.Cu) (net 5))
 (segment (start 178.225 87.122) (end 178.225 81.534) (width 0.6) (layer F.Cu) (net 5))
 (segment (start 178.225 81.534) (end 178.225 81.49) (width 0.6) (layer F.Cu) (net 5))
 (segment (start 179.705 80.01) (end 182.245 80.01) (width 0.6) (layer F.Cu) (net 5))
 (segment (start 178.225 81.49) (end 179.705 80.01) (width 0.6) (layer F.Cu) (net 5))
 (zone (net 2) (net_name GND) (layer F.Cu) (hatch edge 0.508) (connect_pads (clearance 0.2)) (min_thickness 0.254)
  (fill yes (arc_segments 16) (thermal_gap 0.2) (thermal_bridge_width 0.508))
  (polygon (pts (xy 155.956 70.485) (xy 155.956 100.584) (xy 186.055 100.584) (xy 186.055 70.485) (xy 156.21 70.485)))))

